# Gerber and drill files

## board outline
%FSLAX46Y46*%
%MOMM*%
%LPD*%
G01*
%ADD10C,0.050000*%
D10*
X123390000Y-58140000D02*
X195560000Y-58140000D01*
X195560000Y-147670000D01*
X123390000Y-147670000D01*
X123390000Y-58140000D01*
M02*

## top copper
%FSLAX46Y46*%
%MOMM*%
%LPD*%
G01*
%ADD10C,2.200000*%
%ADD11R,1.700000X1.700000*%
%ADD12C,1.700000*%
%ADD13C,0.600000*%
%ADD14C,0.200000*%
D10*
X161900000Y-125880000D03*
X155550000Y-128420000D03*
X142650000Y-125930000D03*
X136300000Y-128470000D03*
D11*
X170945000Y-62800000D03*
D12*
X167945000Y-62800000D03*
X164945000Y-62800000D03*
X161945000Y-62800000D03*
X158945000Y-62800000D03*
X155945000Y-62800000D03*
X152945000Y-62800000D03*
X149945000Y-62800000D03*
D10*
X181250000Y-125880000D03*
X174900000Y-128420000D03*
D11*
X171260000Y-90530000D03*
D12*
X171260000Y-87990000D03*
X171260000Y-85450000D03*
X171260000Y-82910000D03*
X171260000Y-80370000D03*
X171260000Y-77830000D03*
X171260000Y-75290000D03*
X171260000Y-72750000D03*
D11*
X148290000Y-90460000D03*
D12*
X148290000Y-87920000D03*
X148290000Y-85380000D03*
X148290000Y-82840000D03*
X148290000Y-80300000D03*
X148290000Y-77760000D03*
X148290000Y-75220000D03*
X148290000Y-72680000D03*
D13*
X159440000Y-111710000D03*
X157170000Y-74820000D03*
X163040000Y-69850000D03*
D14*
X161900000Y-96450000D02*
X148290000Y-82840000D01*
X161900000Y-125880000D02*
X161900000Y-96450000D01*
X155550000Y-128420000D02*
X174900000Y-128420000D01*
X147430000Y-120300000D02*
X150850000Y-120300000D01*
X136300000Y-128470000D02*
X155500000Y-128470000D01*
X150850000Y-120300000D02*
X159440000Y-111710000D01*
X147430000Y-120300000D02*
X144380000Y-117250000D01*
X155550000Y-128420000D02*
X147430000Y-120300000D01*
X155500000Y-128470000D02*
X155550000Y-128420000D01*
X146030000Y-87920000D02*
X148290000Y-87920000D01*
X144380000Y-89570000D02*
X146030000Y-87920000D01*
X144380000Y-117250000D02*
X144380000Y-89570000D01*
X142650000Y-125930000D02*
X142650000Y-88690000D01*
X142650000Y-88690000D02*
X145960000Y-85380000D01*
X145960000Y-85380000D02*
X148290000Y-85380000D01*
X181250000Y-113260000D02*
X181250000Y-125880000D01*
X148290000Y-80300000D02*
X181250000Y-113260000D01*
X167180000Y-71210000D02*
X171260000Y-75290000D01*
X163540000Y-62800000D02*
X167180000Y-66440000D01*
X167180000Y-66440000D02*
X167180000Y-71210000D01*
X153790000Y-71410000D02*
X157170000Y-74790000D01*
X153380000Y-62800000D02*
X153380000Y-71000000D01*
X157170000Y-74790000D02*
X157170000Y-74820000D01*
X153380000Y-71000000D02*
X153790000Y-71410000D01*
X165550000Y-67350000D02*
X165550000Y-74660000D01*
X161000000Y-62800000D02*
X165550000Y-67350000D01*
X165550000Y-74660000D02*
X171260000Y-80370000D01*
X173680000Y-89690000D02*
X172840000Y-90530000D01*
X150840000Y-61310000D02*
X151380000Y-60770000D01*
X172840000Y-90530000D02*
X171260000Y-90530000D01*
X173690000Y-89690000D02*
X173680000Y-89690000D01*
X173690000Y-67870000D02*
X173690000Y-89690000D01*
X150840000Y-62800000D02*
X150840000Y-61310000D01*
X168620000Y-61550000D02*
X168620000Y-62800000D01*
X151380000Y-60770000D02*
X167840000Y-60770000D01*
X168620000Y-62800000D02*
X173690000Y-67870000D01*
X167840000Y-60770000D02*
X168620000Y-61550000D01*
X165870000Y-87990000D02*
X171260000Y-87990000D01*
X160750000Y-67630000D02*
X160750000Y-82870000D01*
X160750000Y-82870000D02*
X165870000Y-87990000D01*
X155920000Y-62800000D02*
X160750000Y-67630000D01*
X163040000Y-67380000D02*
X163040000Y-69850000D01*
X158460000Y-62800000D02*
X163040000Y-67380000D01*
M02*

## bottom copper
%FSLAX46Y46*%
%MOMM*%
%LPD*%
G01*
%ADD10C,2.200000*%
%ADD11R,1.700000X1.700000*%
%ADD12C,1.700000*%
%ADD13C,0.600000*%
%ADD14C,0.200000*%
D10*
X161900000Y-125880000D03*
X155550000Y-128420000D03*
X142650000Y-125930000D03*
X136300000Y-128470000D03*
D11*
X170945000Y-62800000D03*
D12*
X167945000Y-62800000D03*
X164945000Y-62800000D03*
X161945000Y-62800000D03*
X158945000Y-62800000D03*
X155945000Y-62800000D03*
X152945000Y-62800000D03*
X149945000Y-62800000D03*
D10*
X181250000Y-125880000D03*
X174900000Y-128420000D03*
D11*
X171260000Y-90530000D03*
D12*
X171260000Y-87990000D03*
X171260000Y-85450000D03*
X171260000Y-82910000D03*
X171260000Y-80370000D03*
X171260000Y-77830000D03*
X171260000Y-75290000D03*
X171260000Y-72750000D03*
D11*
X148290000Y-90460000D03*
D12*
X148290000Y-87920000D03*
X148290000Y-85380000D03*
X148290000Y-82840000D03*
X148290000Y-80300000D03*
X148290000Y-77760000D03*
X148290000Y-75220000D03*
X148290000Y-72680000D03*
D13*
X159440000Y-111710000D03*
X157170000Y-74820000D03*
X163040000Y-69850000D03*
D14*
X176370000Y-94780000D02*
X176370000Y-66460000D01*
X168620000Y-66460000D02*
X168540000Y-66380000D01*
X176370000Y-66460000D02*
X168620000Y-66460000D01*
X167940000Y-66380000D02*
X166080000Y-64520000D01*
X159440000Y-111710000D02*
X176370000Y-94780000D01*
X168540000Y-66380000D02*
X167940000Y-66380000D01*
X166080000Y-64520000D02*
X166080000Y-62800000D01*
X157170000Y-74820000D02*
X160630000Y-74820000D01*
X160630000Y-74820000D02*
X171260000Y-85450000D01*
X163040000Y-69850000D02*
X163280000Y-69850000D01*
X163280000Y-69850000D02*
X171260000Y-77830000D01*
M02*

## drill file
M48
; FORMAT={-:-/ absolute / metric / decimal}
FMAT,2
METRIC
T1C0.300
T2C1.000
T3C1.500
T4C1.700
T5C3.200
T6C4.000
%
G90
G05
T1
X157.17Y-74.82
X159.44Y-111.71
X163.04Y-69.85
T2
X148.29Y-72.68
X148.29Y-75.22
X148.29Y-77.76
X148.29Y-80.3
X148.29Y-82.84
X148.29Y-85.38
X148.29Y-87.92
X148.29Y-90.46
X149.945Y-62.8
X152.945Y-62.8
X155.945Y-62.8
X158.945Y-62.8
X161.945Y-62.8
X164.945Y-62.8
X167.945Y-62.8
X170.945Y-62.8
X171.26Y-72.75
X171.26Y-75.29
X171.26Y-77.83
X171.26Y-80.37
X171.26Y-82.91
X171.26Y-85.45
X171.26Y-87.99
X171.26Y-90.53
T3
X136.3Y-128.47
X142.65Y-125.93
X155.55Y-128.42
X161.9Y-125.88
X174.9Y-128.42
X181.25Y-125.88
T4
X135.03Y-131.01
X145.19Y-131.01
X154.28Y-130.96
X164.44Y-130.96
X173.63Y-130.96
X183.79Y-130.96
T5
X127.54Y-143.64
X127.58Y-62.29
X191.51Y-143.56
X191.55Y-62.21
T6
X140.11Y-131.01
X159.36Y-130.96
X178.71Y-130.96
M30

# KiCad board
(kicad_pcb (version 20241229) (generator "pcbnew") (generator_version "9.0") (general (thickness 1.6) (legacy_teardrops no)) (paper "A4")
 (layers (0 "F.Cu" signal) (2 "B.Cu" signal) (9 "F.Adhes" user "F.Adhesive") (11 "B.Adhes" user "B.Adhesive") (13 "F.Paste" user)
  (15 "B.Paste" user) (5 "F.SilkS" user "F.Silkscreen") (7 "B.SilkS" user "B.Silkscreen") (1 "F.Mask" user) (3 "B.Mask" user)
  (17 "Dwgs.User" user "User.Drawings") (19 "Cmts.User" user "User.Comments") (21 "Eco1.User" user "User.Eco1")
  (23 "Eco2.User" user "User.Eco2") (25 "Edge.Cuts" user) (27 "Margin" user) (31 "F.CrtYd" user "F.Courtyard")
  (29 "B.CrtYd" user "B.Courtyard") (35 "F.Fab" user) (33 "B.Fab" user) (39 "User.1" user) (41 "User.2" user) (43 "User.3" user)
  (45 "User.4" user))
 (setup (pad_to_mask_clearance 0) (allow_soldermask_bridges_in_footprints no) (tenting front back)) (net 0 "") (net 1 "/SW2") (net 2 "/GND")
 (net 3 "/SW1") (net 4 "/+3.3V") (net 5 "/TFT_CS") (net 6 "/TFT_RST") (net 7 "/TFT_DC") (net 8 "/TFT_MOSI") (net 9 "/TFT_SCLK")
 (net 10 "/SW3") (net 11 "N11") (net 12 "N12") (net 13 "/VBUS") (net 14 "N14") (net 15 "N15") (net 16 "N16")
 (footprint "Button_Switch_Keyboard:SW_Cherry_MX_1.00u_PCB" (layer "F.Cu") (at 161.9 125.88)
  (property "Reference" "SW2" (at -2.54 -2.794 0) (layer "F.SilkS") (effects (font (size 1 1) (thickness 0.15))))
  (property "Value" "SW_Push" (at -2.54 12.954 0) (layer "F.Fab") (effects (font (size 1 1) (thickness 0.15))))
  (pad "" np_thru_hole circle (at -7.62 5.08) (size 1.7 1.7) (drill 1.7) (layers "*.Cu" "*.Mask"))
  (pad "" np_thru_hole circle (at -2.54 5.08) (size 4 4) (drill 4) (layers "*.Cu" "*.Mask"))
  (pad "" np_thru_hole circle (at 2.54 5.08) (size 1.7 1.7) (drill 1.7) (layers "*.Cu" "*.Mask"))
  (pad "1" thru_hole circle (at 0 0) (size 2.2 2.2) (drill 1.5) (layers "*.Cu" "*.Mask") (remove_unused_layers no) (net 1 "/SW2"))
  (pad "2" thru_hole circle (at -6.35 2.54) (size 2.2 2.2) (drill 1.5) (layers "*.Cu" "*.Mask") (remove_unused_layers no) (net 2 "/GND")))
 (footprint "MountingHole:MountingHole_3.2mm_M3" (layer "F.Cu") (at 191.55 62.21)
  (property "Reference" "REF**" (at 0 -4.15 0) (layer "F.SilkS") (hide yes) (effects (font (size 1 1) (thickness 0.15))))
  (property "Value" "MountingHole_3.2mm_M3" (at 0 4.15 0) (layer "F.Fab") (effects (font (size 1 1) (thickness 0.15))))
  (pad "" np_thru_hole circle (at 0 0) (size 3.2 3.2) (drill 3.2) (layers "*.Cu" "*.Mask")))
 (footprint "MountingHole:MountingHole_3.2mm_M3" (layer "F.Cu") (at 127.54 143.64)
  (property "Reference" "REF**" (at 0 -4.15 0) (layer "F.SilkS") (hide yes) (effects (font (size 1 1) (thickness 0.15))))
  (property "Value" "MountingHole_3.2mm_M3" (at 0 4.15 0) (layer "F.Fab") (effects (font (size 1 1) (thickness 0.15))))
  (pad "" np_thru_hole circle (at 0 0) (size 3.2 3.2) (drill 3.2) (layers "*.Cu" "*.Mask")))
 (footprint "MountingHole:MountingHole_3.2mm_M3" (layer "F.Cu") (at 127.58 62.29)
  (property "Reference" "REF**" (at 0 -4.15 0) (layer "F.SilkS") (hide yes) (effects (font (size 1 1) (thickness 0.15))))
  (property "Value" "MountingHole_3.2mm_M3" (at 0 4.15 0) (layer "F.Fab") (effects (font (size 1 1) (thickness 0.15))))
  (pad "" np_thru_hole circle (at 0 0) (size 3.2 3.2) (drill 3.2) (layers "*.Cu" "*.Mask")))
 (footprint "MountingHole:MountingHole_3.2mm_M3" (layer "F.Cu") (at 191.51 143.56)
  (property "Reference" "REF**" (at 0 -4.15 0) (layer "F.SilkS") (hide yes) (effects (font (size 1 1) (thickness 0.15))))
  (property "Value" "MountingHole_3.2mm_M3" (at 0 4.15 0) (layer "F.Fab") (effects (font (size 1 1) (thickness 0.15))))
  (pad "" np_thru_hole circle (at 0 0) (size 3.2 3.2) (drill 3.2) (layers "*.Cu" "*.Mask")))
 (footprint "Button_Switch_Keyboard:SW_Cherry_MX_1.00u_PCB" (layer "F.Cu") (at 142.65 125.93)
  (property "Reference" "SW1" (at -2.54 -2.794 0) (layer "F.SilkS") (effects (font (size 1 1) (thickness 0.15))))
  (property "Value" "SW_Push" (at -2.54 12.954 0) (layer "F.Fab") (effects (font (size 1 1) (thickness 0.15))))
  (pad "" np_thru_hole circle (at -7.62 5.08) (size 1.7 1.7) (drill 1.7) (layers "*.Cu" "*.Mask"))
  (pad "" np_thru_hole circle (at -2.54 5.08) (size 4 4) (drill 4) (layers "*.Cu" "*.Mask"))
  (pad "" np_thru_hole circle (at 2.54 5.08) (size 1.7 1.7) (drill 1.7) (layers "*.Cu" "*.Mask"))
  (pad "1" thru_hole circle (at 0 0) (size 2.2 2.2) (drill 1.5) (layers "*.Cu" "*.Mask") (remove_unused_layers no) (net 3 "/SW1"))
  (pad "2" thru_hole circle (at -6.35 2.54) (size 2.2 2.2) (drill 1.5) (layers "*.Cu" "*.Mask") (remove_unused_layers no) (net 2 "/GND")))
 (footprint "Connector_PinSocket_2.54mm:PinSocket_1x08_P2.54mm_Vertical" (layer "F.Cu") (at 168.62 62.8 -90)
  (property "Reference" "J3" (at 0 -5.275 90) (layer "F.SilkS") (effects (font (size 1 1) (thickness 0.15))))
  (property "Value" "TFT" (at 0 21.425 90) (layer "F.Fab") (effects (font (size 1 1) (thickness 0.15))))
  (pad "1" thru_hole rect (at 0 -2.325 270) (size 1.7 1.7) (drill 1) (layers "*.Cu" "*.Mask") (remove_unused_layers no) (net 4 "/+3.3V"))
  (pad "2" thru_hole circle (at 0 0.675 270) (size 1.7 1.7) (drill 1) (layers "*.Cu" "*.Mask") (remove_unused_layers no) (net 2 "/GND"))
  (pad "3" thru_hole circle (at 0 3.675 270) (size 1.7 1.7) (drill 1) (layers "*.Cu" "*.Mask") (remove_unused_layers no) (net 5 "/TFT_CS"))
  (pad "4" thru_hole circle (at 0 6.675 270) (size 1.7 1.7) (drill 1) (layers "*.Cu" "*.Mask") (remove_unused_layers no) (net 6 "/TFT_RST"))
  (pad "5" thru_hole circle (at 0 9.675 270) (size 1.7 1.7) (drill 1) (layers "*.Cu" "*.Mask") (remove_unused_layers no) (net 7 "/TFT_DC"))
  (pad "6" thru_hole circle (at 0 12.675 270) (size 1.7 1.7) (drill 1) (layers "*.Cu" "*.Mask") (remove_unused_layers no)
   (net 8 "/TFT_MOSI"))
  (pad "7" thru_hole circle (at 0 15.675 270) (size 1.7 1.7) (drill 1) (layers "*.Cu" "*.Mask") (remove_unused_layers no)
   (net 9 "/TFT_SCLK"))
  (pad "8" thru_hole circle (at 0 18.675 270) (size 1.7 1.7) (drill 1) (layers "*.Cu" "*.Mask") (remove_unused_layers no) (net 4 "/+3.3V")))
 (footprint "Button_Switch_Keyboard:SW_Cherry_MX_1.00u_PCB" (layer "F.Cu") (at 181.25 125.88)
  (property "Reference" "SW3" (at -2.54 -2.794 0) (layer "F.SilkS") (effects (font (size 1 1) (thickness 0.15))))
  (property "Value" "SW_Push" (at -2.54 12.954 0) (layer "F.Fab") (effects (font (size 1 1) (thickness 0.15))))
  (pad "" np_thru_hole circle (at -7.62 5.08) (size 1.7 1.7) (drill 1.7) (layers "*.Cu" "*.Mask"))
  (pad "" np_thru_hole circle (at -2.54 5.08) (size 4 4) (drill 4) (layers "*.Cu" "*.Mask"))
  (pad "" np_thru_hole circle (at 2.54 5.08) (size 1.7 1.7) (drill 1.7) (layers "*.Cu" "*.Mask"))
  (pad "1" thru_hole circle (at 0 0) (size 2.2 2.2) (drill 1.5) (layers "*.Cu" "*.Mask") (remove_unused_layers no) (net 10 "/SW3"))
  (pad "2" thru_hole circle (at -6.35 2.54) (size 2.2 2.2) (drill 1.5) (layers "*.Cu" "*.Mask") (remove_unused_layers no) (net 2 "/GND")))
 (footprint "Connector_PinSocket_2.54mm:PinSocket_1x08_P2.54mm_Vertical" (layer "B.Cu") (at 171.26 90.53)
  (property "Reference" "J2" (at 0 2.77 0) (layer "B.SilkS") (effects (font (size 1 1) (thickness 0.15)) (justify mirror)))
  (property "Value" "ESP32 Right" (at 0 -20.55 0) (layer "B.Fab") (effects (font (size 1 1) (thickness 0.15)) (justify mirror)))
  (pad "1" thru_hole rect (at 0 0) (size 1.7 1.7) (drill 1) (layers "*.Cu" "*.Mask") (remove_unused_layers no) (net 4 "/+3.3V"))
  (pad "2" thru_hole circle (at 0 -2.54) (size 1.7 1.7) (drill 1) (layers "*.Cu" "*.Mask") (remove_unused_layers no) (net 8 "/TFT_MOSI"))
  (pad "3" thru_hole circle (at 0 -5.08) (size 1.7 1.7) (drill 1) (layers "*.Cu" "*.Mask") (remove_unused_layers no) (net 9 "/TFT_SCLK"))
  (pad "4" thru_hole circle (at 0 -7.62) (size 1.7 1.7) (drill 1) (layers "*.Cu" "*.Mask") (remove_unused_layers no) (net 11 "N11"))
  (pad "5" thru_hole circle (at 0 -10.16) (size 1.7 1.7) (drill 1) (layers "*.Cu" "*.Mask") (remove_unused_layers no) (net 6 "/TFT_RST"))
  (pad "6" thru_hole circle (at 0 -12.7) (size 1.7 1.7) (drill 1) (layers "*.Cu" "*.Mask") (remove_unused_layers no) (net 7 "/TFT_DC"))
  (pad "7" thru_hole circle (at 0 -15.24) (size 1.7 1.7) (drill 1) (layers "*.Cu" "*.Mask") (remove_unused_layers no) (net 5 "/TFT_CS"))
  (pad "8" thru_hole circle (at 0 -17.78) (size 1.7 1.7) (drill 1) (layers "*.Cu" "*.Mask") (remove_unused_layers no) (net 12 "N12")))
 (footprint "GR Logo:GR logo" (layer "B.Cu") (at 159.938098 110.253625 180)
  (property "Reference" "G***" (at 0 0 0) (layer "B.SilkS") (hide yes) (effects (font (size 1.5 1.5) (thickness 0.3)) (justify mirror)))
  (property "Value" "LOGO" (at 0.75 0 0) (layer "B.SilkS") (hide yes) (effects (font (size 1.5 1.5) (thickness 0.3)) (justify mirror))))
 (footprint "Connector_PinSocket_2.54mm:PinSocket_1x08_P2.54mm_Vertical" (layer "B.Cu") (at 148.29 90.46)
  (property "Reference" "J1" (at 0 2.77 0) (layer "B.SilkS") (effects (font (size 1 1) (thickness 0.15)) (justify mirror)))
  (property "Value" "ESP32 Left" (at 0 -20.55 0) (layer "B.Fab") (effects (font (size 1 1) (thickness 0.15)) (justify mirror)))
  (pad "1" thru_hole rect (at 0 0) (size 1.7 1.7) (drill 1) (layers "*.Cu" "*.Mask") (remove_unused_layers no) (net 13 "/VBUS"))
  (pad "2" thru_hole circle (at 0 -2.54) (size 1.7 1.7) (drill 1) (layers "*.Cu" "*.Mask") (remove_unused_layers no) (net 2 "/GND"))
  (pad "3" thru_hole circle (at 0 -5.08) (size 1.7 1.7) (drill 1) (layers "*.Cu" "*.Mask") (remove_unused_layers no) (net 3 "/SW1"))
  (pad "4" thru_hole circle (at 0 -7.62) (size 1.7 1.7) (drill 1) (layers "*.Cu" "*.Mask") (remove_unused_layers no) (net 1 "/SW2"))
  (pad "5" thru_hole circle (at 0 -10.16) (size 1.7 1.7) (drill 1) (layers "*.Cu" "*.Mask") (remove_unused_layers no) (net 10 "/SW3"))
  (pad "6" thru_hole circle (at 0 -12.7) (size 1.7 1.7) (drill 1) (layers "*.Cu" "*.Mask") (remove_unused_layers no) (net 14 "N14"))
  (pad "7" thru_hole circle (at 0 -15.24) (size 1.7 1.7) (drill 1) (layers "*.Cu" "*.Mask") (remove_unused_layers no) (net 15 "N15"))
  (pad "8" thru_hole circle (at 0 -17.78) (size 1.7 1.7) (drill 1) (layers "*.Cu" "*.Mask") (remove_unused_layers no) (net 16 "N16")))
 (gr_rect (start 123.39 58.14) (end 195.56 147.67) (stroke (width 0.05) (type default)) (fill no) (layer "Edge.Cuts"))
 (segment (start 161.9 96.45) (end 148.29 82.84) (width 0.2) (layer "F.Cu") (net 1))
 (segment (start 161.9 125.88) (end 161.9 96.45) (width 0.2) (layer "F.Cu") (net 1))
 (segment (start 155.55 128.42) (end 174.9 128.42) (width 0.2) (layer "F.Cu") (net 2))
 (segment (start 147.43 120.3) (end 150.85 120.3) (width 0.2) (layer "F.Cu") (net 2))
 (segment (start 136.3 128.47) (end 155.5 128.47) (width 0.2) (layer "F.Cu") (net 2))
 (segment (start 150.85 120.3) (end 159.44 111.71) (width 0.2) (layer "F.Cu") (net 2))
 (segment (start 147.43 120.3) (end 144.38 117.25) (width 0.2) (layer "F.Cu") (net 2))
 (segment (start 155.55 128.42) (end 147.43 120.3) (width 0.2) (layer "F.Cu") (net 2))
 (segment (start 155.5 128.47) (end 155.55 128.42) (width 0.2) (layer "F.Cu") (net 2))
 (segment (start 146.03 87.92) (end 148.29 87.92) (width 0.2) (layer "F.Cu") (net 2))
 (segment (start 144.38 89.57) (end 146.03 87.92) (width 0.2) (layer "F.Cu") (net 2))
 (segment (start 144.38 117.25) (end 144.38 89.57) (width 0.2) (layer "F.Cu") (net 2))
 (via (at 159.44 111.71) (size 0.6) (drill 0.3) (layers "F.Cu" "B.Cu") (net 2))
 (segment (start 176.37 94.78) (end 176.37 66.46) (width 0.2) (layer "B.Cu") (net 2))
 (segment (start 168.62 66.46) (end 168.54 66.38) (width 0.2) (layer "B.Cu") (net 2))
 (segment (start 176.37 66.46) (end 168.62 66.46) (width 0.2) (layer "B.Cu") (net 2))
 (segment (start 167.94 66.38) (end 166.08 64.52) (width 0.2) (layer "B.Cu") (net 2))
 (segment (start 159.44 111.71) (end 176.37 94.78) (width 0.2) (layer "B.Cu") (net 2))
 (segment (start 168.54 66.38) (end 167.94 66.38) (width 0.2) (layer "B.Cu") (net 2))
 (segment (start 166.08 64.52) (end 166.08 62.8) (width 0.2) (layer "B.Cu") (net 2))
 (segment (start 142.65 125.93) (end 142.65 88.69) (width 0.2) (layer "F.Cu") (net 3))
 (segment (start 142.65 88.69) (end 145.96 85.38) (width 0.2) (layer "F.Cu") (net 3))
 (segment (start 145.96 85.38) (end 148.29 85.38) (width 0.2) (layer "F.Cu") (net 3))
 (segment (start 181.25 113.26) (end 181.25 125.88) (width 0.2) (layer "F.Cu") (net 10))
 (segment (start 148.29 80.3) (end 181.25 113.26) (width 0.2) (layer "F.Cu") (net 10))
 (segment (start 167.18 71.21) (end 171.26 75.29) (width 0.2) (layer "F.Cu") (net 5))
 (segment (start 163.54 62.8) (end 167.18 66.44) (width 0.2) (layer "F.Cu") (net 5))
 (segment (start 167.18 66.44) (end 167.18 71.21) (width 0.2) (layer "F.Cu") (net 5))
 (segment (start 153.79 71.41) (end 157.17 74.79) (width 0.2) (layer "F.Cu") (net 9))
 (segment (start 153.38 62.8) (end 153.38 71) (width 0.2) (layer "F.Cu") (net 9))
 (segment (start 157.17 74.79) (end 157.17 74.82) (width 0.2) (layer "F.Cu") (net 9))
 (segment (start 153.38 71) (end 153.79 71.41) (width 0.2) (layer "F.Cu") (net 9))
 (via (at 157.17 74.82) (size 0.6) (drill 0.3) (layers "F.Cu" "B.Cu") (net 9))
 (segment (start 157.17 74.82) (end 160.63 74.82) (width 0.2) (layer "B.Cu") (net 9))
 (segment (start 160.63 74.82) (end 171.26 85.45) (width 0.2) (layer "B.Cu") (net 9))
 (segment (start 165.55 67.35) (end 165.55 74.66) (width 0.2) (layer "F.Cu") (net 6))
 (segment (start 161 62.8) (end 165.55 67.35) (width 0.2) (layer "F.Cu") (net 6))
 (segment (start 165.55 74.66) (end 171.26 80.37) (width 0.2) (layer "F.Cu") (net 6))
 (segment (start 173.68 89.69) (end 172.84 90.53) (width 0.2) (layer "F.Cu") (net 4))
 (segment (start 150.84 61.31) (end 151.38 60.77) (width 0.2) (layer "F.Cu") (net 4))
 (segment (start 172.84 90.53) (end 171.26 90.53) (width 0.2) (layer "F.Cu") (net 4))
 (segment (start 173.69 89.69) (end 173.68 89.69) (width 0.2) (layer "F.Cu") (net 4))
 (segment (start 173.69 67.87) (end 173.69 89.69) (width 0.2) (layer "F.Cu") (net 4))
 (segment (start 150.84 62.8) (end 150.84 61.31) (width 0.2) (layer "F.Cu") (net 4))
 (segment (start 168.62 61.55) (end 168.62 62.8) (width 0.2) (layer "F.Cu") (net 4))
 (segment (start 151.38 60.77) (end 167.84 60.77) (width 0.2) (layer "F.Cu") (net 4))
 (segment (start 168.62 62.8) (end 173.69 67.87) (width 0.2) (layer "F.Cu") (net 4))
 (segment (start 167.84 60.77) (end 168.62 61.55) (width 0.2) (layer "F.Cu") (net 4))
 (segment (start 165.87 87.99) (end 171.26 87.99) (width 0.2) (layer "F.Cu") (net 8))
 (segment (start 160.75 67.63) (end 160.75 82.87) (width 0.2) (layer "F.Cu") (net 8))
 (segment (start 160.75 82.87) (end 165.87 87.99) (width 0.2) (layer "F.Cu") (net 8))
 (segment (start 155.92 62.8) (end 160.75 67.63) (width 0.2) (layer "F.Cu") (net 8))
 (segment (start 163.04 67.38) (end 163.04 69.85) (width 0.2) (layer "F.Cu") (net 7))
 (segment (start 158.46 62.8) (end 163.04 67.38) (width 0.2) (layer "F.Cu") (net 7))
 (via (at 163.04 69.85) (size 0.6) (drill 0.3) (layers "F.Cu" "B.Cu") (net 7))
 (segment (start 163.04 69.85) (end 163.28 69.85) (width 0.2) (layer "B.Cu") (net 7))
 (segment (start 163.28 69.85) (end 171.26 77.83) (width 0.2) (layer "B.Cu") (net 7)))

